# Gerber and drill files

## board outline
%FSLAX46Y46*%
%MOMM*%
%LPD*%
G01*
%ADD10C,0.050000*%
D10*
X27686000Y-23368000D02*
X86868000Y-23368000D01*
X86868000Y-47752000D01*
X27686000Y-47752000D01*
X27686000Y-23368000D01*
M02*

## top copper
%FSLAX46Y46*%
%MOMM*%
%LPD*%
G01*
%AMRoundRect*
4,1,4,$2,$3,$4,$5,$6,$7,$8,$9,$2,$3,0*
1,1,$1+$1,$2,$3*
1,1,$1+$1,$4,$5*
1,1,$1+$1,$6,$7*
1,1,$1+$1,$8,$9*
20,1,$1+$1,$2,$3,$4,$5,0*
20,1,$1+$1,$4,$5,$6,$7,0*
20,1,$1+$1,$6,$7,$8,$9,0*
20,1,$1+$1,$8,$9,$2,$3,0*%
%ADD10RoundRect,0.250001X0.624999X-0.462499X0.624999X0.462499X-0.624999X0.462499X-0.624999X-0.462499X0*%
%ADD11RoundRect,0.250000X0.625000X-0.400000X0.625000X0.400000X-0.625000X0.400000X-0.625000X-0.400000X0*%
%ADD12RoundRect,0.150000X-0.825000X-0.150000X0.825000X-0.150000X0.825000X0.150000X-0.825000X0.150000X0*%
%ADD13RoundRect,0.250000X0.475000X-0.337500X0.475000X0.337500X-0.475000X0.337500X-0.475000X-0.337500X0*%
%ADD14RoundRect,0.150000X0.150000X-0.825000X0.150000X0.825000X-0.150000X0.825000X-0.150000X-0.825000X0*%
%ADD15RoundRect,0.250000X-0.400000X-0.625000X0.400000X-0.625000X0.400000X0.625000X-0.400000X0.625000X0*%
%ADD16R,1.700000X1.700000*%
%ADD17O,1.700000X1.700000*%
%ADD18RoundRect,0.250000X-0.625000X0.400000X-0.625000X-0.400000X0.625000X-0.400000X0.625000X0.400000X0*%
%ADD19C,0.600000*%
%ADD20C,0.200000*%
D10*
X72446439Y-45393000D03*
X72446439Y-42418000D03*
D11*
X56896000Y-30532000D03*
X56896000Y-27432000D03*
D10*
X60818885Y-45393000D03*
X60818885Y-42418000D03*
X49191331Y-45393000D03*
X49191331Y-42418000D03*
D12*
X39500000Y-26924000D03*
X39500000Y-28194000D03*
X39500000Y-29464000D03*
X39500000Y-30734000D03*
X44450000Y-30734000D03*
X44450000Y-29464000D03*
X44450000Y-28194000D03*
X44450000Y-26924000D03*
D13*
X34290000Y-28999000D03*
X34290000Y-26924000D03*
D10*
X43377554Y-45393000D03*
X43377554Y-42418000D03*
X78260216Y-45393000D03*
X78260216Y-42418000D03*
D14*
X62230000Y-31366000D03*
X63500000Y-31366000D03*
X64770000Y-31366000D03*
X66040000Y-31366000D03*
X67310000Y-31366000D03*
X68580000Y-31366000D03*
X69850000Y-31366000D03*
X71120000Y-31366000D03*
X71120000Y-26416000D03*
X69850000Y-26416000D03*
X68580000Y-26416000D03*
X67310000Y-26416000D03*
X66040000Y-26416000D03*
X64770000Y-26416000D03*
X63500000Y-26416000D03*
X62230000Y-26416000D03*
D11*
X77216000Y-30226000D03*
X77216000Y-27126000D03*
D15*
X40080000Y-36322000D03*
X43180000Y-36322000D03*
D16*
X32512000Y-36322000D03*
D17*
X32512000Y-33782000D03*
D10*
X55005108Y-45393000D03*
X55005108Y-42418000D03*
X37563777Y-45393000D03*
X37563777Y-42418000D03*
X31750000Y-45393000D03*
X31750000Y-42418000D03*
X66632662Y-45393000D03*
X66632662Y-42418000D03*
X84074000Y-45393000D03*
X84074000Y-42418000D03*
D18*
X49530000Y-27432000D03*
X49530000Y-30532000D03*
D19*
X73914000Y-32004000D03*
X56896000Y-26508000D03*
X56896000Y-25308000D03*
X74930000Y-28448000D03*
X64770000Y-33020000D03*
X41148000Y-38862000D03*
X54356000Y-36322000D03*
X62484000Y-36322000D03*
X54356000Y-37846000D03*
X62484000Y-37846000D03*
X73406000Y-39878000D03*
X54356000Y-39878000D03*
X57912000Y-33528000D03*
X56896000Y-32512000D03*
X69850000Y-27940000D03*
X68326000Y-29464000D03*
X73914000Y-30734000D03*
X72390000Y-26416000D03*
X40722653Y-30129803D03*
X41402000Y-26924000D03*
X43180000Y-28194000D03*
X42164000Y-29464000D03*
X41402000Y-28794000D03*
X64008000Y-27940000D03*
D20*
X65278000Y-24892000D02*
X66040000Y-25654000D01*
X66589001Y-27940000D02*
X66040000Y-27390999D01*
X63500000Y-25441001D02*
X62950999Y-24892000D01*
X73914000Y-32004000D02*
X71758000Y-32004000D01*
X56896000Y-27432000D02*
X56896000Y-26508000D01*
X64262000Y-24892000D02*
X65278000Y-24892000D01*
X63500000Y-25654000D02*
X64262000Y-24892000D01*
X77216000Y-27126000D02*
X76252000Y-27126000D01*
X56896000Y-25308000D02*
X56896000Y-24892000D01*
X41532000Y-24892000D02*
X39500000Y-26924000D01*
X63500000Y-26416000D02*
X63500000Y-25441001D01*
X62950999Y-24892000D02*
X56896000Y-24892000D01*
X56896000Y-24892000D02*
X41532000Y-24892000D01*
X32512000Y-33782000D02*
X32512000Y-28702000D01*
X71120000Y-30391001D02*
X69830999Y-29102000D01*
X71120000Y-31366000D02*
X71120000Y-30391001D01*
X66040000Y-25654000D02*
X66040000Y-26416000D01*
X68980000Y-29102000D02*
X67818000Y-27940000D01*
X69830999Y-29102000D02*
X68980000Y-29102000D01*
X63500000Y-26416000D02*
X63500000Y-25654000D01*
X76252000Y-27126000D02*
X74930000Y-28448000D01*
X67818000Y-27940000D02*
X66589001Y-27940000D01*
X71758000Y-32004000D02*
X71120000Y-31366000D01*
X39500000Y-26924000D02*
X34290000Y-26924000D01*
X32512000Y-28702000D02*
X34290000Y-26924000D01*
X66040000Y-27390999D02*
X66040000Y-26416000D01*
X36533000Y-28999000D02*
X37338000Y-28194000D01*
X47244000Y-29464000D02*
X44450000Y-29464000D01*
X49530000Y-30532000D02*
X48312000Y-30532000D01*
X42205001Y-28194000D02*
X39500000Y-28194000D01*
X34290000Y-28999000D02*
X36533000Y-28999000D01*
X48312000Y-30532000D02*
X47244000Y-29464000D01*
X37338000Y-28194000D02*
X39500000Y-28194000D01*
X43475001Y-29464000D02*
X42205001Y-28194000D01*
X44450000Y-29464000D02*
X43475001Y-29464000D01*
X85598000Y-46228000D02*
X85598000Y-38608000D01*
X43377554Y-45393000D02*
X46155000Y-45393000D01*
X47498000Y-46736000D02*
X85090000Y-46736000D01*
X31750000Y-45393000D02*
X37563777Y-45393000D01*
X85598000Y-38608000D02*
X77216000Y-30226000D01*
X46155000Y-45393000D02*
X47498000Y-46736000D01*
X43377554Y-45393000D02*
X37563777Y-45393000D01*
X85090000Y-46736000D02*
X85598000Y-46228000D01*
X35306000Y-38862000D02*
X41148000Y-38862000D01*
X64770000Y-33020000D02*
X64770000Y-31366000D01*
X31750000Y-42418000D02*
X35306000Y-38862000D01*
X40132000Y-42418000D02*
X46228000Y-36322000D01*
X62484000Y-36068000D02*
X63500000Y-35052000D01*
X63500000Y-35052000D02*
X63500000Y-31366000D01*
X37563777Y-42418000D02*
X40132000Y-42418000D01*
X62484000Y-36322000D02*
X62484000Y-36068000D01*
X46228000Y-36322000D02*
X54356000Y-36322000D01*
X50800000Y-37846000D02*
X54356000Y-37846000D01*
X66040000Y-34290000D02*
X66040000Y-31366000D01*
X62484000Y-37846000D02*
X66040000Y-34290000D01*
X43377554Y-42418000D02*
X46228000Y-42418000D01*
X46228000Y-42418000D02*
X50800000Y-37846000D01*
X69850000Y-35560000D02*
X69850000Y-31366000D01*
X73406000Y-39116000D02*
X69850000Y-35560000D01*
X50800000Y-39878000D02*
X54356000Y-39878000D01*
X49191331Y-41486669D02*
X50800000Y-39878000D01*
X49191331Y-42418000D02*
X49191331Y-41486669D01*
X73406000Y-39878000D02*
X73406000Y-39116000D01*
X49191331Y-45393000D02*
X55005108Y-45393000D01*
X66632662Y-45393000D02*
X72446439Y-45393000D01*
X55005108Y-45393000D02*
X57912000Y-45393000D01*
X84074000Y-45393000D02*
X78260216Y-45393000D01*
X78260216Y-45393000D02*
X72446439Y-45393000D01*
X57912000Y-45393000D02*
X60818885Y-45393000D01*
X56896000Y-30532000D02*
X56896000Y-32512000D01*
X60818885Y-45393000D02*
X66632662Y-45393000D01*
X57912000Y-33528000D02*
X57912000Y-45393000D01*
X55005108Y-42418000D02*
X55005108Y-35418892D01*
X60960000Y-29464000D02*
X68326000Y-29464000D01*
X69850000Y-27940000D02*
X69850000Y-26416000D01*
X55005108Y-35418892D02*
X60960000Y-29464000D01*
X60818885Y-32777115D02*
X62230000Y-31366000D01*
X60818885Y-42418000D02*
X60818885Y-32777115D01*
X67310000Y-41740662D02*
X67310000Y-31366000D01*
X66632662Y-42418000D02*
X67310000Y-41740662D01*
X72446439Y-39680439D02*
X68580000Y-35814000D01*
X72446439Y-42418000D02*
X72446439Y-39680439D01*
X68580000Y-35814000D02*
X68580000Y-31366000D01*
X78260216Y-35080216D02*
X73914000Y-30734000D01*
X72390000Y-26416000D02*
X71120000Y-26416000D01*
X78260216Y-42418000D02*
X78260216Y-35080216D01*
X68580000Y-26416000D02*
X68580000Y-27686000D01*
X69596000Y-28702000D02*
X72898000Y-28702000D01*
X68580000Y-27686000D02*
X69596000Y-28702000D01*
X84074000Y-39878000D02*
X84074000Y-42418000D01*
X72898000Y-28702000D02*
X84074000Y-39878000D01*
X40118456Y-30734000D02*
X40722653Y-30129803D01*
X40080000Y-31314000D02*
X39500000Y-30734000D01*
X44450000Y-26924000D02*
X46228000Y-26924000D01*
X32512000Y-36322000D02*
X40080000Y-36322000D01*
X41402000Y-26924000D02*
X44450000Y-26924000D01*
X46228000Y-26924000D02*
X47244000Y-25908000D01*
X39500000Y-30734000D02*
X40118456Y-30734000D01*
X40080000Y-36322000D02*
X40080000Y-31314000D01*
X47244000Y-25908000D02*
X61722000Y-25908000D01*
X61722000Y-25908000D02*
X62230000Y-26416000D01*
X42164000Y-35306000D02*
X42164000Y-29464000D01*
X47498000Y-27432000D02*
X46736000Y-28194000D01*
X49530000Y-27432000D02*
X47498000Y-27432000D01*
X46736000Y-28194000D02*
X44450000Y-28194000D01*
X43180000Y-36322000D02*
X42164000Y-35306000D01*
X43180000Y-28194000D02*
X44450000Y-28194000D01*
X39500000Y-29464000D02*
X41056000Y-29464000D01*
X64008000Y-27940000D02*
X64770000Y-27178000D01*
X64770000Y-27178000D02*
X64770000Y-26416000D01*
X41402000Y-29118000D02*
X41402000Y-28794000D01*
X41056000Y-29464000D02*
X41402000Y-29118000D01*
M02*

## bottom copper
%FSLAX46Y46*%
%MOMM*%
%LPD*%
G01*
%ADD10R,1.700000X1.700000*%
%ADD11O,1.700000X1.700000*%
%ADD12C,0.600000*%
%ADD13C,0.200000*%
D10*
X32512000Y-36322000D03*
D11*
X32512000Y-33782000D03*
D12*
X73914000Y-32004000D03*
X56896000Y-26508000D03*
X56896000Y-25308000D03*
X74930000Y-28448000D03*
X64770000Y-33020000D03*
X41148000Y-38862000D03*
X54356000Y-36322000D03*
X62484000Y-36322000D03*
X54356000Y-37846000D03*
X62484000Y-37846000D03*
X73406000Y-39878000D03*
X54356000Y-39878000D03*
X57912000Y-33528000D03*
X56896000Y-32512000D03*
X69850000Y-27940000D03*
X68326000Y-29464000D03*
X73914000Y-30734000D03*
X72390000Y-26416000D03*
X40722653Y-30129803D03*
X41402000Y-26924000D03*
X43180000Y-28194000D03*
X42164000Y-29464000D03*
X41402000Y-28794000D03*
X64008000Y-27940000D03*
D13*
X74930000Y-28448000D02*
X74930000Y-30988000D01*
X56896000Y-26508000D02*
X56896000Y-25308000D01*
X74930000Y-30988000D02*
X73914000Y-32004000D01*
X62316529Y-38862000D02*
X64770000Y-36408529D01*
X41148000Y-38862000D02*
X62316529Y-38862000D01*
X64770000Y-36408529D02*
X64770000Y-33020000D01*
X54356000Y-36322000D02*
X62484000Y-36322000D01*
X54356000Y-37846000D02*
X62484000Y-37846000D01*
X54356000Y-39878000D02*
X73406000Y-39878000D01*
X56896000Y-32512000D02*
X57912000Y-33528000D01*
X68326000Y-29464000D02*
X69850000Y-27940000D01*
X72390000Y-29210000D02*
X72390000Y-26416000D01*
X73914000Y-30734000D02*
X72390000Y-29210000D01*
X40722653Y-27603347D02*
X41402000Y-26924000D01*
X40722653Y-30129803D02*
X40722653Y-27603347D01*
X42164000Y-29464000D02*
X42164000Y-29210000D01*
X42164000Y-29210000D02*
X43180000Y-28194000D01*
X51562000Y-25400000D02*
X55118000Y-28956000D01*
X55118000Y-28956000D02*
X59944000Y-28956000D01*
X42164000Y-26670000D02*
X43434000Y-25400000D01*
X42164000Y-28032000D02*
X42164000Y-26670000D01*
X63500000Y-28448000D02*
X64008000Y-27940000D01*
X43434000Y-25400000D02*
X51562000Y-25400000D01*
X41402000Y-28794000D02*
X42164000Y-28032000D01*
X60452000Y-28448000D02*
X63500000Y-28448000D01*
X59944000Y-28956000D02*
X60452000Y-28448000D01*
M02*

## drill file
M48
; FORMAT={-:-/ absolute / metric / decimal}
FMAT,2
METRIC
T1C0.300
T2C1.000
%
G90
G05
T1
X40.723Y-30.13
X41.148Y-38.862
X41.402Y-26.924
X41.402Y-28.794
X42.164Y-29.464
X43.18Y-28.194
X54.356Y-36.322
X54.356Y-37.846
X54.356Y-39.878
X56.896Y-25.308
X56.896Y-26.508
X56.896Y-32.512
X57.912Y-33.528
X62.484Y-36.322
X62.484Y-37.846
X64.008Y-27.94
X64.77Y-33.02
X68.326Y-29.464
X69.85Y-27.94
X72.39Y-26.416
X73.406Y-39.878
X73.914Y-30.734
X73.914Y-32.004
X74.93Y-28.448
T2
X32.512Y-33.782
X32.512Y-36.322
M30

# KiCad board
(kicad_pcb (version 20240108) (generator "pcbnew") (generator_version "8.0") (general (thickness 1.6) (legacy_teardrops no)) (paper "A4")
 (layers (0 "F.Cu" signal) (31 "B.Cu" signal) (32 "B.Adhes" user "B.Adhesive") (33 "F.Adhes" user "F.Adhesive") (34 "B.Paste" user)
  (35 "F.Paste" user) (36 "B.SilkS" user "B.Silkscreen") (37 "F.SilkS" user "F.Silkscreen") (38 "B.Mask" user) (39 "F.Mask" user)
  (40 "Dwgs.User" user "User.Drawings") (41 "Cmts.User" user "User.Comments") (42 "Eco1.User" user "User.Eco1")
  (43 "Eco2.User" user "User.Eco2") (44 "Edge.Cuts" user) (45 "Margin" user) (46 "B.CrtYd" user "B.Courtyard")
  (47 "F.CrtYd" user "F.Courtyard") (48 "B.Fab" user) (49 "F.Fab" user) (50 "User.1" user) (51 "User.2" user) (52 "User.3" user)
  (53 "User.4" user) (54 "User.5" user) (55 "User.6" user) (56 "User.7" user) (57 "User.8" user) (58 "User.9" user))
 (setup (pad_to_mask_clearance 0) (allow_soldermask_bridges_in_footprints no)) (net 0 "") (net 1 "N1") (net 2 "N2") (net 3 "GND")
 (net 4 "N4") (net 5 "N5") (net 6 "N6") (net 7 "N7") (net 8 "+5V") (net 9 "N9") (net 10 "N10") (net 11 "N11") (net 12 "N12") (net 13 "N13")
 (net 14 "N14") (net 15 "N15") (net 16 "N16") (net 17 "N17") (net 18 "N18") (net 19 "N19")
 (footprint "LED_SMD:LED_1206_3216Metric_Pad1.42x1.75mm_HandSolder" (layer "F.Cu") (at 72.446439 43.9055 90)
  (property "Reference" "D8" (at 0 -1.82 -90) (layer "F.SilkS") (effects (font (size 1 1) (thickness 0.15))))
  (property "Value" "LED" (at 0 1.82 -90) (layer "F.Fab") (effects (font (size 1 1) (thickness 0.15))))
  (pad "1" smd roundrect (at -1.4875 0 90) (size 1.425 1.75) (layers "F.Cu" "F.Paste" "F.Mask") (roundrect_rratio 0.175439) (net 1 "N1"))
  (pad "2" smd roundrect (at 1.4875 0 90) (size 1.425 1.75) (layers "F.Cu" "F.Paste" "F.Mask") (roundrect_rratio 0.175439) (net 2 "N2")))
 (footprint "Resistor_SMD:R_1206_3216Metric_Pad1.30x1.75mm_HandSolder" (layer "F.Cu") (at 56.896 28.982 90)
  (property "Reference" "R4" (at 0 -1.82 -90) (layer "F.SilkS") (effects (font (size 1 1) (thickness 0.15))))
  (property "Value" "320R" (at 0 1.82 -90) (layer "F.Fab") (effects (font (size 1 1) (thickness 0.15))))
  (pad "1" smd roundrect (at -1.55 0 90) (size 1.3 1.75) (layers "F.Cu" "F.Paste" "F.Mask") (roundrect_rratio 0.192308) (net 1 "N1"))
  (pad "2" smd roundrect (at 1.55 0 90) (size 1.3 1.75) (layers "F.Cu" "F.Paste" "F.Mask") (roundrect_rratio 0.192308) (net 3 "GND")))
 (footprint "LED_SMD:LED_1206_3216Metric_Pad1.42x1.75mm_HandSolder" (layer "F.Cu") (at 60.818885 43.9055 90)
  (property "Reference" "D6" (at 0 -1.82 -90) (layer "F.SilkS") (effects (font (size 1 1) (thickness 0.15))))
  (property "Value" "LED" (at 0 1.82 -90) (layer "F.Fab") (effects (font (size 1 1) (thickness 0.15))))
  (pad "1" smd roundrect (at -1.4875 0 90) (size 1.425 1.75) (layers "F.Cu" "F.Paste" "F.Mask") (roundrect_rratio 0.175439) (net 1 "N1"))
  (pad "2" smd roundrect (at 1.4875 0 90) (size 1.425 1.75) (layers "F.Cu" "F.Paste" "F.Mask") (roundrect_rratio 0.175439) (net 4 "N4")))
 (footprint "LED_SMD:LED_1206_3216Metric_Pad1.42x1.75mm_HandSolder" (layer "F.Cu") (at 49.191331 43.9055 90)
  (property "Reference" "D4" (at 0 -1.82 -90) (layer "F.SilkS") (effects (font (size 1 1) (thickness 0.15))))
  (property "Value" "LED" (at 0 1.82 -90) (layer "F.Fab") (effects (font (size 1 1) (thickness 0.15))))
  (pad "1" smd roundrect (at -1.4875 0 90) (size 1.425 1.75) (layers "F.Cu" "F.Paste" "F.Mask") (roundrect_rratio 0.175439) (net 1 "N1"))
  (pad "2" smd roundrect (at 1.4875 0 90) (size 1.425 1.75) (layers "F.Cu" "F.Paste" "F.Mask") (roundrect_rratio 0.175439) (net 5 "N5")))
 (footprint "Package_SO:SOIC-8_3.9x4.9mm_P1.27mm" (layer "F.Cu") (at 41.975 28.829)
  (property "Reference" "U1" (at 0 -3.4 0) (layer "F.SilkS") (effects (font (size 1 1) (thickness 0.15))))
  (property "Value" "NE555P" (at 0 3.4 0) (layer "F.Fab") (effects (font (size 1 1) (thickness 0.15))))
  (pad "1" smd roundrect (at -2.475 -1.905) (size 1.95 0.6) (layers "F.Cu" "F.Paste" "F.Mask") (roundrect_rratio 0.25) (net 3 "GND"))
  (pad "2" smd roundrect (at -2.475 -0.635) (size 1.95 0.6) (layers "F.Cu" "F.Paste" "F.Mask") (roundrect_rratio 0.25) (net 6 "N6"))
  (pad "3" smd roundrect (at -2.475 0.635) (size 1.95 0.6) (layers "F.Cu" "F.Paste" "F.Mask") (roundrect_rratio 0.25) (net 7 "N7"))
  (pad "4" smd roundrect (at -2.475 1.905) (size 1.95 0.6) (layers "F.Cu" "F.Paste" "F.Mask") (roundrect_rratio 0.25) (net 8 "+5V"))
  (pad "5" smd roundrect (at 2.475 1.905) (size 1.95 0.6) (layers "F.Cu" "F.Paste" "F.Mask") (roundrect_rratio 0.25) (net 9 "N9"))
  (pad "6" smd roundrect (at 2.475 0.635) (size 1.95 0.6) (layers "F.Cu" "F.Paste" "F.Mask") (roundrect_rratio 0.25) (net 6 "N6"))
  (pad "7" smd roundrect (at 2.475 -0.635) (size 1.95 0.6) (layers "F.Cu" "F.Paste" "F.Mask") (roundrect_rratio 0.25) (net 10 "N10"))
  (pad "8" smd roundrect (at 2.475 -1.905) (size 1.95 0.6) (layers "F.Cu" "F.Paste" "F.Mask") (roundrect_rratio 0.25) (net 8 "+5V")))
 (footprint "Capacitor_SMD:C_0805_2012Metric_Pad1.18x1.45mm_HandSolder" (layer "F.Cu") (at 34.29 27.9615 90)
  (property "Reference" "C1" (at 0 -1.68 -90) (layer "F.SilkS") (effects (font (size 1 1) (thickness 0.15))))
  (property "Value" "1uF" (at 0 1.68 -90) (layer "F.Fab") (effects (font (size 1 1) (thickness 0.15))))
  (pad "1" smd roundrect (at -1.0375 0 90) (size 1.175 1.45) (layers "F.Cu" "F.Paste" "F.Mask") (roundrect_rratio 0.212766) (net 6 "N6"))
  (pad "2" smd roundrect (at 1.0375 0 90) (size 1.175 1.45) (layers "F.Cu" "F.Paste" "F.Mask") (roundrect_rratio 0.212766) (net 3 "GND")))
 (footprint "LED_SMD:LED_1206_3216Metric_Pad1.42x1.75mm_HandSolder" (layer "F.Cu") (at 43.377554 43.9055 90)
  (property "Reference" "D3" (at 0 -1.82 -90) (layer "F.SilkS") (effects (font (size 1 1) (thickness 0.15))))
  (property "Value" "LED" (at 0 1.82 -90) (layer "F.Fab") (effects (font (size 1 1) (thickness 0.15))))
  (pad "1" smd roundrect (at -1.4875 0 90) (size 1.425 1.75) (layers "F.Cu" "F.Paste" "F.Mask") (roundrect_rratio 0.175439) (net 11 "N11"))
  (pad "2" smd roundrect (at 1.4875 0 90) (size 1.425 1.75) (layers "F.Cu" "F.Paste" "F.Mask") (roundrect_rratio 0.175439) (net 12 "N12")))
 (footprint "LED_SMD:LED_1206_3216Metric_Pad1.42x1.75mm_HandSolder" (layer "F.Cu") (at 78.260216 43.9055 90)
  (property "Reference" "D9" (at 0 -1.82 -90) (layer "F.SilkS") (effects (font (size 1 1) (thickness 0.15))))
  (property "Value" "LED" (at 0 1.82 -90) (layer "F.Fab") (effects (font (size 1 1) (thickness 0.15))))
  (pad "1" smd roundrect (at -1.4875 0 90) (size 1.425 1.75) (layers "F.Cu" "F.Paste" "F.Mask") (roundrect_rratio 0.175439) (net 1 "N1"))
  (pad "2" smd roundrect (at 1.4875 0 90) (size 1.425 1.75) (layers "F.Cu" "F.Paste" "F.Mask") (roundrect_rratio 0.175439) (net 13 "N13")))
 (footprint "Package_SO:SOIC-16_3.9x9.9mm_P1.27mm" (layer "F.Cu") (at 66.675 28.891 90)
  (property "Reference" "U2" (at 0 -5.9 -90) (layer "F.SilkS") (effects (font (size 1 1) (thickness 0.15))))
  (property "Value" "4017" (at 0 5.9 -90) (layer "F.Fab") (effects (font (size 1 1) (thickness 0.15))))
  (pad "1" smd roundrect (at -2.475 -4.445 90) (size 1.95 0.6) (layers "F.Cu" "F.Paste" "F.Mask") (roundrect_rratio 0.25) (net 4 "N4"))
  (pad "2" smd roundrect (at -2.475 -3.175 90) (size 1.95 0.6) (layers "F.Cu" "F.Paste" "F.Mask") (roundrect_rratio 0.25) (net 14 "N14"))
  (pad "3" smd roundrect (at -2.475 -1.905 90) (size 1.95 0.6) (layers "F.Cu" "F.Paste" "F.Mask") (roundrect_rratio 0.25) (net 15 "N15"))
  (pad "4" smd roundrect (at -2.475 -0.635 90) (size 1.95 0.6) (layers "F.Cu" "F.Paste" "F.Mask") (roundrect_rratio 0.25) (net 12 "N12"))
  (pad "5" smd roundrect (at -2.475 0.635 90) (size 1.95 0.6) (layers "F.Cu" "F.Paste" "F.Mask") (roundrect_rratio 0.25) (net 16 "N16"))
  (pad "6" smd roundrect (at -2.475 1.905 90) (size 1.95 0.6) (layers "F.Cu" "F.Paste" "F.Mask") (roundrect_rratio 0.25) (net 2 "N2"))
  (pad "7" smd roundrect (at -2.475 3.175 90) (size 1.95 0.6) (layers "F.Cu" "F.Paste" "F.Mask") (roundrect_rratio 0.25) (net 5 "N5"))
  (pad "8" smd roundrect (at -2.475 4.445 90) (size 1.95 0.6) (layers "F.Cu" "F.Paste" "F.Mask") (roundrect_rratio 0.25) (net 3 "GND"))
  (pad "9" smd roundrect (at 2.475 4.445 90) (size 1.95 0.6) (layers "F.Cu" "F.Paste" "F.Mask") (roundrect_rratio 0.25) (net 13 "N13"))
  (pad "10" smd roundrect (at 2.475 3.175 90) (size 1.95 0.6) (layers "F.Cu" "F.Paste" "F.Mask") (roundrect_rratio 0.25) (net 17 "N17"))
  (pad "11" smd roundrect (at 2.475 1.905 90) (size 1.95 0.6) (layers "F.Cu" "F.Paste" "F.Mask") (roundrect_rratio 0.25) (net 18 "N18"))
  (pad "12" smd roundrect (at 2.475 0.635 90) (size 1.95 0.6) (layers "F.Cu" "F.Paste" "F.Mask") (roundrect_rratio 0.25) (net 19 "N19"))
  (pad "13" smd roundrect (at 2.475 -0.635 90) (size 1.95 0.6) (layers "F.Cu" "F.Paste" "F.Mask") (roundrect_rratio 0.25) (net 3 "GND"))
  (pad "14" smd roundrect (at 2.475 -1.905 90) (size 1.95 0.6) (layers "F.Cu" "F.Paste" "F.Mask") (roundrect_rratio 0.25) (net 7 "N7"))
  (pad "15" smd roundrect (at 2.475 -3.175 90) (size 1.95 0.6) (layers "F.Cu" "F.Paste" "F.Mask") (roundrect_rratio 0.25) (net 3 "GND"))
  (pad "16" smd roundrect (at 2.475 -4.445 90) (size 1.95 0.6) (layers "F.Cu" "F.Paste" "F.Mask") (roundrect_rratio 0.25) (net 8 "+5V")))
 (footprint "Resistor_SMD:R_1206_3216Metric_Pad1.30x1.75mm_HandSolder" (layer "F.Cu") (at 77.216 28.676 90)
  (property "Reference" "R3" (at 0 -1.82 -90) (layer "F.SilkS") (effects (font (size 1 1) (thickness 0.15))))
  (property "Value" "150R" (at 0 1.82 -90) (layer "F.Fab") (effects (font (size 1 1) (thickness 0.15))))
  (pad "1" smd roundrect (at -1.55 0 90) (size 1.3 1.75) (layers "F.Cu" "F.Paste" "F.Mask") (roundrect_rratio 0.192308) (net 11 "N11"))
  (pad "2" smd roundrect (at 1.55 0 90) (size 1.3 1.75) (layers "F.Cu" "F.Paste" "F.Mask") (roundrect_rratio 0.192308) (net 3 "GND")))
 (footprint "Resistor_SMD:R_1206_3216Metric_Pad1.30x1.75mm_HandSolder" (layer "F.Cu") (at 41.63 36.322)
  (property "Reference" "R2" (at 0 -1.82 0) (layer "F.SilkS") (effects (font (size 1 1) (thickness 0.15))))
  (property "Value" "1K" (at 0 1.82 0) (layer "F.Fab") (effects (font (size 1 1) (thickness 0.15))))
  (pad "1" smd roundrect (at -1.55 0) (size 1.3 1.75) (layers "F.Cu" "F.Paste" "F.Mask") (roundrect_rratio 0.192308) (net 8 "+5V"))
  (pad "2" smd roundrect (at 1.55 0) (size 1.3 1.75) (layers "F.Cu" "F.Paste" "F.Mask") (roundrect_rratio 0.192308) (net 10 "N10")))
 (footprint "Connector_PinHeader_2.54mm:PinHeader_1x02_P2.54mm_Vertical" (layer "F.Cu") (at 32.512 36.322 180)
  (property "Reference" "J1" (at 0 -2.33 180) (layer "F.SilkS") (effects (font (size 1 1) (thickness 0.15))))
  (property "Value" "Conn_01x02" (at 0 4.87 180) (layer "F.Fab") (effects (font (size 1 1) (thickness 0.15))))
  (pad "1" thru_hole rect (at 0 0 180) (size 1.7 1.7) (drill 1) (layers "*.Cu" "*.Mask") (remove_unused_layers no) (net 8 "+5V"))
  (pad "2" thru_hole oval (at 0 2.54 180) (size 1.7 1.7) (drill 1) (layers "*.Cu" "*.Mask") (remove_unused_layers no) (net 3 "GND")))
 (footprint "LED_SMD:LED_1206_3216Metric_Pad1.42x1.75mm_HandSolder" (layer "F.Cu") (at 55.005108 43.9055 90)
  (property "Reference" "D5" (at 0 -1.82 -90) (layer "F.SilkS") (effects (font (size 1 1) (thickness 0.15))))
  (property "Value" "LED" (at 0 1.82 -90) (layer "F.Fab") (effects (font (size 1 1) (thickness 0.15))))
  (pad "1" smd roundrect (at -1.4875 0 90) (size 1.425 1.75) (layers "F.Cu" "F.Paste" "F.Mask") (roundrect_rratio 0.175439) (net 1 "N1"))
  (pad "2" smd roundrect (at 1.4875 0 90) (size 1.425 1.75) (layers "F.Cu" "F.Paste" "F.Mask") (roundrect_rratio 0.175439) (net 17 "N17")))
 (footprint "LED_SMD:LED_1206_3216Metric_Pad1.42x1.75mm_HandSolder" (layer "F.Cu") (at 37.563777 43.9055 90)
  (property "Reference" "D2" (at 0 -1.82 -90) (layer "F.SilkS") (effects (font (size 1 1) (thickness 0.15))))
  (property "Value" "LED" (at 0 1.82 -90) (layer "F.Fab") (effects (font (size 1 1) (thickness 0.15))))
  (pad "1" smd roundrect (at -1.4875 0 90) (size 1.425 1.75) (layers "F.Cu" "F.Paste" "F.Mask") (roundrect_rratio 0.175439) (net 11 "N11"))
  (pad "2" smd roundrect (at 1.4875 0 90) (size 1.425 1.75) (layers "F.Cu" "F.Paste" "F.Mask") (roundrect_rratio 0.175439) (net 14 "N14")))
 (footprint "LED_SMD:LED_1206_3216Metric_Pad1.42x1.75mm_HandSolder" (layer "F.Cu") (at 31.75 43.9055 90)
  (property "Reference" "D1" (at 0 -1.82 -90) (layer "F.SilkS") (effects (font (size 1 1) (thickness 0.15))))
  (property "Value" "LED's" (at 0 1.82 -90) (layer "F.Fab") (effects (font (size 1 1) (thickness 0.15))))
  (pad "1" smd roundrect (at -1.4875 0 90) (size 1.425 1.75) (layers "F.Cu" "F.Paste" "F.Mask") (roundrect_rratio 0.175439) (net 11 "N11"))
  (pad "2" smd roundrect (at 1.4875 0 90) (size 1.425 1.75) (layers "F.Cu" "F.Paste" "F.Mask") (roundrect_rratio 0.175439) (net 15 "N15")))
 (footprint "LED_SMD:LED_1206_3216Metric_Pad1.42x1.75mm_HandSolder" (layer "F.Cu") (at 66.632662 43.9055 90)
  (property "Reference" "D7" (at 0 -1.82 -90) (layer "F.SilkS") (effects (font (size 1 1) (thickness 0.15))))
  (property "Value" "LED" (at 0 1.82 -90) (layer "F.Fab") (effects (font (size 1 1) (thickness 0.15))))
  (pad "1" smd roundrect (at -1.4875 0 90) (size 1.425 1.75) (layers "F.Cu" "F.Paste" "F.Mask") (roundrect_rratio 0.175439) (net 1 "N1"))
  (pad "2" smd roundrect (at 1.4875 0 90) (size 1.425 1.75) (layers "F.Cu" "F.Paste" "F.Mask") (roundrect_rratio 0.175439) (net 16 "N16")))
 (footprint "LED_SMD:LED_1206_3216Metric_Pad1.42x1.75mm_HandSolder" (layer "F.Cu") (at 84.074 43.9055 90)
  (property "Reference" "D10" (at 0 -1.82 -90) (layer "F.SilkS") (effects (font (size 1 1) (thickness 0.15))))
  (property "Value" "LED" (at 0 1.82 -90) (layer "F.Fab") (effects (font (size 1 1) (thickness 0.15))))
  (pad "1" smd roundrect (at -1.4875 0 90) (size 1.425 1.75) (layers "F.Cu" "F.Paste" "F.Mask") (roundrect_rratio 0.175439) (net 1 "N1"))
  (pad "2" smd roundrect (at 1.4875 0 90) (size 1.425 1.75) (layers "F.Cu" "F.Paste" "F.Mask") (roundrect_rratio 0.175439) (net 18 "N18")))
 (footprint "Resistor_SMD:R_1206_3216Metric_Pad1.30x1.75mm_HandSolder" (layer "F.Cu") (at 49.53 28.982 -90)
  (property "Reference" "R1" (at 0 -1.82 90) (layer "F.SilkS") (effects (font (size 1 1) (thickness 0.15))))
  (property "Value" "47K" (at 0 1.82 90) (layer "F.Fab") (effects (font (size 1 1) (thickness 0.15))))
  (pad "1" smd roundrect (at -1.55 0 270) (size 1.3 1.75) (layers "F.Cu" "F.Paste" "F.Mask") (roundrect_rratio 0.192308) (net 10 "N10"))
  (pad "2" smd roundrect (at 1.55 0 270) (size 1.3 1.75) (layers "F.Cu" "F.Paste" "F.Mask") (roundrect_rratio 0.192308) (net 6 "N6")))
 (gr_rect (start 27.686 23.368) (end 86.868 47.752) (stroke (width 0.05) (type default)) (fill none) (layer "Edge.Cuts"))
 (segment (start 65.278 24.892) (end 66.04 25.654) (width 0.2) (layer "F.Cu") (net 3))
 (segment (start 66.589001 27.94) (end 66.04 27.390999) (width 0.2) (layer "F.Cu") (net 3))
 (segment (start 63.5 25.441001) (end 62.950999 24.892) (width 0.2) (layer "F.Cu") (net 3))
 (segment (start 73.914 32.004) (end 71.758 32.004) (width 0.2) (layer "F.Cu") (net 3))
 (segment (start 56.896 27.432) (end 56.896 26.508) (width 0.2) (layer "F.Cu") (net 3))
 (segment (start 64.262 24.892) (end 65.278 24.892) (width 0.2) (layer "F.Cu") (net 3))
 (segment (start 63.5 25.654) (end 64.262 24.892) (width 0.2) (layer "F.Cu") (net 3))
 (segment (start 77.216 27.126) (end 76.252 27.126) (width 0.2) (layer "F.Cu") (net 3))
 (segment (start 56.896 25.308) (end 56.896 24.892) (width 0.2) (layer "F.Cu") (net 3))
 (segment (start 41.532 24.892) (end 39.5 26.924) (width 0.2) (layer "F.Cu") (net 3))
 (segment (start 63.5 26.416) (end 63.5 25.441001) (width 0.2) (layer "F.Cu") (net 3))
 (segment (start 62.950999 24.892) (end 56.896 24.892) (width 0.2) (layer "F.Cu") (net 3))
 (segment (start 56.896 24.892) (end 41.532 24.892) (width 0.2) (layer "F.Cu") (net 3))
 (segment (start 32.512 33.782) (end 32.512 28.702) (width 0.2) (layer "F.Cu") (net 3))
 (segment (start 71.12 30.391001) (end 69.830999 29.102) (width 0.2) (layer "F.Cu") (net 3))
 (segment (start 71.12 31.366) (end 71.12 30.391001) (width 0.2) (layer "F.Cu") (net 3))
 (segment (start 66.04 25.654) (end 66.04 26.416) (width 0.2) (layer "F.Cu") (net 3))
 (segment (start 68.98 29.102) (end 67.818 27.94) (width 0.2) (layer "F.Cu") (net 3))
 (segment (start 69.830999 29.102) (end 68.98 29.102) (width 0.2) (layer "F.Cu") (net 3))
 (segment (start 63.5 26.416) (end 63.5 25.654) (width 0.2) (layer "F.Cu") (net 3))
 (segment (start 76.252 27.126) (end 74.93 28.448) (width 0.2) (layer "F.Cu") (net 3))
 (segment (start 67.818 27.94) (end 66.589001 27.94) (width 0.2) (layer "F.Cu") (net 3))
 (segment (start 71.758 32.004) (end 71.12 31.366) (width 0.2) (layer "F.Cu") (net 3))
 (segment (start 39.5 26.924) (end 34.29 26.924) (width 0.2) (layer "F.Cu") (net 3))
 (segment (start 32.512 28.702) (end 34.29 26.924) (width 0.2) (layer "F.Cu") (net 3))
 (segment (start 66.04 27.390999) (end 66.04 26.416) (width 0.2) (layer "F.Cu") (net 3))
 (via (at 73.914 32.004) (size 0.6) (drill 0.3) (layers "F.Cu" "B.Cu") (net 3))
 (via (at 56.896 26.508) (size 0.6) (drill 0.3) (layers "F.Cu" "B.Cu") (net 3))
 (via (at 56.896 25.308) (size 0.6) (drill 0.3) (layers "F.Cu" "B.Cu") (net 3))
 (via (at 74.93 28.448) (size 0.6) (drill 0.3) (layers "F.Cu" "B.Cu") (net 3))
 (segment (start 74.93 28.448) (end 74.93 30.988) (width 0.2) (layer "B.Cu") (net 3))
 (segment (start 56.896 26.508) (end 56.896 25.308) (width 0.2) (layer "B.Cu") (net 3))
 (segment (start 74.93 30.988) (end 73.914 32.004) (width 0.2) (layer "B.Cu") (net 3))
 (segment (start 36.533 28.999) (end 37.338 28.194) (width 0.2) (layer "F.Cu") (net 6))
 (segment (start 47.244 29.464) (end 44.45 29.464) (width 0.2) (layer "F.Cu") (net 6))
 (segment (start 49.53 30.532) (end 48.312 30.532) (width 0.2) (layer "F.Cu") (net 6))
 (segment (start 42.205001 28.194) (end 39.5 28.194) (width 0.2) (layer "F.Cu") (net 6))
 (segment (start 34.29 28.999) (end 36.533 28.999) (width 0.2) (layer "F.Cu") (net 6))
 (segment (start 48.312 30.532) (end 47.244 29.464) (width 0.2) (layer "F.Cu") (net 6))
 (segment (start 37.338 28.194) (end 39.5 28.194) (width 0.2) (layer "F.Cu") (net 6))
 (segment (start 43.475001 29.464) (end 42.205001 28.194) (width 0.2) (layer "F.Cu") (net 6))
 (segment (start 44.45 29.464) (end 43.475001 29.464) (width 0.2) (layer "F.Cu") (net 6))
 (segment (start 85.598 46.228) (end 85.598 38.608) (width 0.2) (layer "F.Cu") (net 11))
 (segment (start 43.377554 45.393) (end 46.155 45.393) (width 0.2) (layer "F.Cu") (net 11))
 (segment (start 47.498 46.736) (end 85.09 46.736) (width 0.2) (layer "F.Cu") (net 11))
 (segment (start 31.75 45.393) (end 37.563777 45.393) (width 0.2) (layer "F.Cu") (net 11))
 (segment (start 85.598 38.608) (end 77.216 30.226) (width 0.2) (layer "F.Cu") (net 11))
 (segment (start 46.155 45.393) (end 47.498 46.736) (width 0.2) (layer "F.Cu") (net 11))
 (segment (start 43.377554 45.393) (end 37.563777 45.393) (width 0.2) (layer "F.Cu") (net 11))
 (segment (start 85.09 46.736) (end 85.598 46.228) (width 0.2) (layer "F.Cu") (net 11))
 (segment (start 35.306 38.862) (end 41.148 38.862) (width 0.2) (layer "F.Cu") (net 15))
 (segment (start 64.77 33.02) (end 64.77 31.366) (width 0.2) (layer "F.Cu") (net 15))
 (segment (start 31.75 42.418) (end 35.306 38.862) (width 0.2) (layer "F.Cu") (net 15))
 (via (at 64.77 33.02) (size 0.6) (drill 0.3) (layers "F.Cu" "B.Cu") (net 15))
 (via (at 41.148 38.862) (size 0.6) (drill 0.3) (layers "F.Cu" "B.Cu") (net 15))
 (segment (start 62.316529 38.862) (end 64.77 36.408529) (width 0.2) (layer "B.Cu") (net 15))
 (segment (start 41.148 38.862) (end 62.316529 38.862) (width 0.2) (layer "B.Cu") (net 15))
 (segment (start 64.77 36.408529) (end 64.77 33.02) (width 0.2) (layer "B.Cu") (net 15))
 (segment (start 40.132 42.418) (end 46.228 36.322) (width 0.2) (layer "F.Cu") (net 14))
 (segment (start 62.484 36.068) (end 63.5 35.052) (width 0.2) (layer "F.Cu") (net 14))
 (segment (start 63.5 35.052) (end 63.5 31.366) (width 0.2) (layer "F.Cu") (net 14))
 (segment (start 37.563777 42.418) (end 40.132 42.418) (width 0.2) (layer "F.Cu") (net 14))
 (segment (start 62.484 36.322) (end 62.484 36.068) (width 0.2) (layer "F.Cu") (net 14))
 (segment (start 46.228 36.322) (end 54.356 36.322) (width 0.2) (layer "F.Cu") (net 14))
 (via (at 54.356 36.322) (size 0.6) (drill 0.3) (layers "F.Cu" "B.Cu") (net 14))
 (via (at 62.484 36.322) (size 0.6) (drill 0.3) (layers "F.Cu" "B.Cu") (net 14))
 (segment (start 54.356 36.322) (end 62.484 36.322) (width 0.2) (layer "B.Cu") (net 14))
 (segment (start 50.8 37.846) (end 54.356 37.846) (width 0.2) (layer "F.Cu") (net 12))
 (segment (start 66.04 34.29) (end 66.04 31.366) (width 0.2) (layer "F.Cu") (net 12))
 (segment (start 62.484 37.846) (end 66.04 34.29) (width 0.2) (layer "F.Cu") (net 12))
 (segment (start 43.377554 42.418) (end 46.228 42.418) (width 0.2) (layer "F.Cu") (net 12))
 (segment (start 46.228 42.418) (end 50.8 37.846) (width 0.2) (layer "F.Cu") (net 12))
 (via (at 54.356 37.846) (size 0.6) (drill 0.3) (layers "F.Cu" "B.Cu") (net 12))
 (via (at 62.484 37.846) (size 0.6) (drill 0.3) (layers "F.Cu" "B.Cu") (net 12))
 (segment (start 54.356 37.846) (end 62.484 37.846) (width 0.2) (layer "B.Cu") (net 12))
 (segment (start 69.85 35.56) (end 69.85 31.366) (width 0.2) (layer "F.Cu") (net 5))
 (segment (start 73.406 39.116) (end 69.85 35.56) (width 0.2) (layer "F.Cu") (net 5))
 (segment (start 50.8 39.878) (end 54.356 39.878) (width 0.2) (layer "F.Cu") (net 5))
 (segment (start 49.191331 41.486669) (end 50.8 39.878) (width 0.2) (layer "F.Cu") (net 5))
 (segment (start 49.191331 42.418) (end 49.191331 41.486669) (width 0.2) (layer "F.Cu") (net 5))
 (segment (start 73.406 39.878) (end 73.406 39.116) (width 0.2) (layer "F.Cu") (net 5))
 (via (at 73.406 39.878) (size 0.6) (drill 0.3) (layers "F.Cu" "B.Cu") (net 5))
 (via (at 54.356 39.878) (size 0.6) (drill 0.3) (layers "F.Cu" "B.Cu") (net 5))
 (segment (start 54.356 39.878) (end 73.406 39.878) (width 0.2) (layer "B.Cu") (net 5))
 (segment (start 49.191331 45.393) (end 55.005108 45.393) (width 0.2) (layer "F.Cu") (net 1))
 (segment (start 66.632662 45.393) (end 72.446439 45.393) (width 0.2) (layer "F.Cu") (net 1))
 (segment (start 55.005108 45.393) (end 57.912 45.393) (width 0.2) (layer "F.Cu") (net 1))
 (segment (start 84.074 45.393) (end 78.260216 45.393) (width 0.2) (layer "F.Cu") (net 1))
 (segment (start 78.260216 45.393) (end 72.446439 45.393) (width 0.2) (layer "F.Cu") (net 1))
 (segment (start 57.912 45.393) (end 60.818885 45.393) (width 0.2) (layer "F.Cu") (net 1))
 (segment (start 56.896 30.532) (end 56.896 32.512) (width 0.2) (layer "F.Cu") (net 1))
 (segment (start 60.818885 45.393) (end 66.632662 45.393) (width 0.2) (layer "F.Cu") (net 1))
 (segment (start 57.912 33.528) (end 57.912 45.393) (width 0.2) (layer "F.Cu") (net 1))
 (via (at 57.912 33.528) (size 0.6) (drill 0.3) (layers "F.Cu" "B.Cu") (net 1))
 (via (at 56.896 32.512) (size 0.6) (drill 0.3) (layers "F.Cu" "B.Cu") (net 1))
 (segment (start 56.896 32.512) (end 57.912 33.528) (width 0.2) (layer "B.Cu") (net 1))
 (segment (start 55.005108 42.418) (end 55.005108 35.418892) (width 0.2) (layer "F.Cu") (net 17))
 (segment (start 60.96 29.464) (end 68.326 29.464) (width 0.2) (layer "F.Cu") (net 17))
 (segment (start 69.85 27.94) (end 69.85 26.416) (width 0.2) (layer "F.Cu") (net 17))
 (segment (start 55.005108 35.418892) (end 60.96 29.464) (width 0.2) (layer "F.Cu") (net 17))
 (via (at 69.85 27.94) (size 0.6) (drill 0.3) (layers "F.Cu" "B.Cu") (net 17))
 (via (at 68.326 29.464) (size 0.6) (drill 0.3) (layers "F.Cu" "B.Cu") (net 17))
 (segment (start 68.326 29.464) (end 69.85 27.94) (width 0.2) (layer "B.Cu") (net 17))
 (segment (start 60.818885 32.777115) (end 62.23 31.366) (width 0.2) (layer "F.Cu") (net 4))
 (segment (start 60.818885 42.418) (end 60.818885 32.777115) (width 0.2) (layer "F.Cu") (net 4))
 (segment (start 67.31 41.740662) (end 67.31 31.366) (width 0.2) (layer "F.Cu") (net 16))
 (segment (start 66.632662 42.418) (end 67.31 41.740662) (width 0.2) (layer "F.Cu") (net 16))
 (segment (start 72.446439 39.680439) (end 68.58 35.814) (width 0.2) (layer "F.Cu") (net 2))
 (segment (start 72.446439 42.418) (end 72.446439 39.680439) (width 0.2) (layer "F.Cu") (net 2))
 (segment (start 68.58 35.814) (end 68.58 31.366) (width 0.2) (layer "F.Cu") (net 2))
 (segment (start 78.260216 35.080216) (end 73.914 30.734) (width 0.2) (layer "F.Cu") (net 13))
 (segment (start 72.39 26.416) (end 71.12 26.416) (width 0.2) (layer "F.Cu") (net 13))
 (segment (start 78.260216 42.418) (end 78.260216 35.080216) (width 0.2) (layer "F.Cu") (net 13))
 (via (at 73.914 30.734) (size 0.6) (drill 0.3) (layers "F.Cu" "B.Cu") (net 13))
 (via (at 72.39 26.416) (size 0.6) (drill 0.3) (layers "F.Cu" "B.Cu") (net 13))
 (segment (start 72.39 29.21) (end 72.39 26.416) (width 0.2) (layer "B.Cu") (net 13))
 (segment (start 73.914 30.734) (end 72.39 29.21) (width 0.2) (layer "B.Cu") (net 13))
 (segment (start 68.58 26.416) (end 68.58 27.686) (width 0.2) (layer "F.Cu") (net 18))
 (segment (start 69.596 28.702) (end 72.898 28.702) (width 0.2) (layer "F.Cu") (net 18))
 (segment (start 68.58 27.686) (end 69.596 28.702) (width 0.2) (layer "F.Cu") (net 18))
 (segment (start 84.074 39.878) (end 84.074 42.418) (width 0.2) (layer "F.Cu") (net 18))
 (segment (start 72.898 28.702) (end 84.074 39.878) (width 0.2) (layer "F.Cu") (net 18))
 (segment (start 40.118456 30.734) (end 40.722653 30.129803) (width 0.2) (layer "F.Cu") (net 8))
 (segment (start 40.08 31.314) (end 39.5 30.734) (width 0.2) (layer "F.Cu") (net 8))
 (segment (start 44.45 26.924) (end 46.228 26.924) (width 0.2) (layer "F.Cu") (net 8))
 (segment (start 32.512 36.322) (end 40.08 36.322) (width 0.2) (layer "F.Cu") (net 8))
 (segment (start 41.402 26.924) (end 44.45 26.924) (width 0.2) (layer "F.Cu") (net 8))
 (segment (start 46.228 26.924) (end 47.244 25.908) (width 0.2) (layer "F.Cu") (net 8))
 (segment (start 39.5 30.734) (end 40.118456 30.734) (width 0.2) (layer "F.Cu") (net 8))
 (segment (start 40.08 36.322) (end 40.08 31.314) (width 0.2) (layer "F.Cu") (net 8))
 (segment (start 47.244 25.908) (end 61.722 25.908) (width 0.2) (layer "F.Cu") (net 8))
 (segment (start 61.722 25.908) (end 62.23 26.416) (width 0.2) (layer "F.Cu") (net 8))
 (via (at 40.722653 30.129803) (size 0.6) (drill 0.3) (layers "F.Cu" "B.Cu") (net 8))
 (via (at 41.402 26.924) (size 0.6) (drill 0.3) (layers "F.Cu" "B.Cu") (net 8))
 (segment (start 40.722653 27.603347) (end 41.402 26.924) (width 0.2) (layer "B.Cu") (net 8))
 (segment (start 40.722653 30.129803) (end 40.722653 27.603347) (width 0.2) (layer "B.Cu") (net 8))
 (segment (start 42.164 35.306) (end 42.164 29.464) (width 0.2) (layer "F.Cu") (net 10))
 (segment (start 47.498 27.432) (end 46.736 28.194) (width 0.2) (layer "F.Cu") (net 10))
 (segment (start 49.53 27.432) (end 47.498 27.432) (width 0.2) (layer "F.Cu") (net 10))
 (segment (start 46.736 28.194) (end 44.45 28.194) (width 0.2) (layer "F.Cu") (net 10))
 (segment (start 43.18 36.322) (end 42.164 35.306) (width 0.2) (layer "F.Cu") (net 10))
 (segment (start 43.18 28.194) (end 44.45 28.194) (width 0.2) (layer "F.Cu") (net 10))
 (via (at 43.18 28.194) (size 0.6) (drill 0.3) (layers "F.Cu" "B.Cu") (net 10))
 (via (at 42.164 29.464) (size 0.6) (drill 0.3) (layers "F.Cu" "B.Cu") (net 10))
 (segment (start 42.164 29.464) (end 42.164 29.21) (width 0.2) (layer "B.Cu") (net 10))
 (segment (start 42.164 29.21) (end 43.18 28.194) (width 0.2) (layer "B.Cu") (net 10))
 (segment (start 39.5 29.464) (end 41.056 29.464) (width 0.2) (layer "F.Cu") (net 7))
 (segment (start 64.008 27.94) (end 64.77 27.178) (width 0.2) (layer "F.Cu") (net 7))
 (segment (start 64.77 27.178) (end 64.77 26.416) (width 0.2) (layer "F.Cu") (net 7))
 (segment (start 41.402 29.118) (end 41.402 28.794) (width 0.2) (layer "F.Cu") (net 7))
 (segment (start 41.056 29.464) (end 41.402 29.118) (width 0.2) (layer "F.Cu") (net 7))
 (via (at 41.402 28.794) (size 0.6) (drill 0.3) (layers "F.Cu" "B.Cu") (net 7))
 (via (at 64.008 27.94) (size 0.6) (drill 0.3) (layers "F.Cu" "B.Cu") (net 7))
 (segment (start 51.562 25.4) (end 55.118 28.956) (width 0.2) (layer "B.Cu") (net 7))
 (segment (start 55.118 28.956) (end 59.944 28.956) (width 0.2) (layer "B.Cu") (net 7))
 (segment (start 42.164 26.67) (end 43.434 25.4) (width 0.2) (layer "B.Cu") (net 7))
 (segment (start 42.164 28.032) (end 42.164 26.67) (width 0.2) (layer "B.Cu") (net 7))
 (segment (start 63.5 28.448) (end 64.008 27.94) (width 0.2) (layer "B.Cu") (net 7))
 (segment (start 43.434 25.4) (end 51.562 25.4) (width 0.2) (layer "B.Cu") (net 7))
 (segment (start 41.402 28.794) (end 42.164 28.032) (width 0.2) (layer "B.Cu") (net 7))
 (segment (start 60.452 28.448) (end 63.5 28.448) (width 0.2) (layer "B.Cu") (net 7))
 (segment (start 59.944 28.956) (end 60.452 28.448) (width 0.2) (layer "B.Cu") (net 7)))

